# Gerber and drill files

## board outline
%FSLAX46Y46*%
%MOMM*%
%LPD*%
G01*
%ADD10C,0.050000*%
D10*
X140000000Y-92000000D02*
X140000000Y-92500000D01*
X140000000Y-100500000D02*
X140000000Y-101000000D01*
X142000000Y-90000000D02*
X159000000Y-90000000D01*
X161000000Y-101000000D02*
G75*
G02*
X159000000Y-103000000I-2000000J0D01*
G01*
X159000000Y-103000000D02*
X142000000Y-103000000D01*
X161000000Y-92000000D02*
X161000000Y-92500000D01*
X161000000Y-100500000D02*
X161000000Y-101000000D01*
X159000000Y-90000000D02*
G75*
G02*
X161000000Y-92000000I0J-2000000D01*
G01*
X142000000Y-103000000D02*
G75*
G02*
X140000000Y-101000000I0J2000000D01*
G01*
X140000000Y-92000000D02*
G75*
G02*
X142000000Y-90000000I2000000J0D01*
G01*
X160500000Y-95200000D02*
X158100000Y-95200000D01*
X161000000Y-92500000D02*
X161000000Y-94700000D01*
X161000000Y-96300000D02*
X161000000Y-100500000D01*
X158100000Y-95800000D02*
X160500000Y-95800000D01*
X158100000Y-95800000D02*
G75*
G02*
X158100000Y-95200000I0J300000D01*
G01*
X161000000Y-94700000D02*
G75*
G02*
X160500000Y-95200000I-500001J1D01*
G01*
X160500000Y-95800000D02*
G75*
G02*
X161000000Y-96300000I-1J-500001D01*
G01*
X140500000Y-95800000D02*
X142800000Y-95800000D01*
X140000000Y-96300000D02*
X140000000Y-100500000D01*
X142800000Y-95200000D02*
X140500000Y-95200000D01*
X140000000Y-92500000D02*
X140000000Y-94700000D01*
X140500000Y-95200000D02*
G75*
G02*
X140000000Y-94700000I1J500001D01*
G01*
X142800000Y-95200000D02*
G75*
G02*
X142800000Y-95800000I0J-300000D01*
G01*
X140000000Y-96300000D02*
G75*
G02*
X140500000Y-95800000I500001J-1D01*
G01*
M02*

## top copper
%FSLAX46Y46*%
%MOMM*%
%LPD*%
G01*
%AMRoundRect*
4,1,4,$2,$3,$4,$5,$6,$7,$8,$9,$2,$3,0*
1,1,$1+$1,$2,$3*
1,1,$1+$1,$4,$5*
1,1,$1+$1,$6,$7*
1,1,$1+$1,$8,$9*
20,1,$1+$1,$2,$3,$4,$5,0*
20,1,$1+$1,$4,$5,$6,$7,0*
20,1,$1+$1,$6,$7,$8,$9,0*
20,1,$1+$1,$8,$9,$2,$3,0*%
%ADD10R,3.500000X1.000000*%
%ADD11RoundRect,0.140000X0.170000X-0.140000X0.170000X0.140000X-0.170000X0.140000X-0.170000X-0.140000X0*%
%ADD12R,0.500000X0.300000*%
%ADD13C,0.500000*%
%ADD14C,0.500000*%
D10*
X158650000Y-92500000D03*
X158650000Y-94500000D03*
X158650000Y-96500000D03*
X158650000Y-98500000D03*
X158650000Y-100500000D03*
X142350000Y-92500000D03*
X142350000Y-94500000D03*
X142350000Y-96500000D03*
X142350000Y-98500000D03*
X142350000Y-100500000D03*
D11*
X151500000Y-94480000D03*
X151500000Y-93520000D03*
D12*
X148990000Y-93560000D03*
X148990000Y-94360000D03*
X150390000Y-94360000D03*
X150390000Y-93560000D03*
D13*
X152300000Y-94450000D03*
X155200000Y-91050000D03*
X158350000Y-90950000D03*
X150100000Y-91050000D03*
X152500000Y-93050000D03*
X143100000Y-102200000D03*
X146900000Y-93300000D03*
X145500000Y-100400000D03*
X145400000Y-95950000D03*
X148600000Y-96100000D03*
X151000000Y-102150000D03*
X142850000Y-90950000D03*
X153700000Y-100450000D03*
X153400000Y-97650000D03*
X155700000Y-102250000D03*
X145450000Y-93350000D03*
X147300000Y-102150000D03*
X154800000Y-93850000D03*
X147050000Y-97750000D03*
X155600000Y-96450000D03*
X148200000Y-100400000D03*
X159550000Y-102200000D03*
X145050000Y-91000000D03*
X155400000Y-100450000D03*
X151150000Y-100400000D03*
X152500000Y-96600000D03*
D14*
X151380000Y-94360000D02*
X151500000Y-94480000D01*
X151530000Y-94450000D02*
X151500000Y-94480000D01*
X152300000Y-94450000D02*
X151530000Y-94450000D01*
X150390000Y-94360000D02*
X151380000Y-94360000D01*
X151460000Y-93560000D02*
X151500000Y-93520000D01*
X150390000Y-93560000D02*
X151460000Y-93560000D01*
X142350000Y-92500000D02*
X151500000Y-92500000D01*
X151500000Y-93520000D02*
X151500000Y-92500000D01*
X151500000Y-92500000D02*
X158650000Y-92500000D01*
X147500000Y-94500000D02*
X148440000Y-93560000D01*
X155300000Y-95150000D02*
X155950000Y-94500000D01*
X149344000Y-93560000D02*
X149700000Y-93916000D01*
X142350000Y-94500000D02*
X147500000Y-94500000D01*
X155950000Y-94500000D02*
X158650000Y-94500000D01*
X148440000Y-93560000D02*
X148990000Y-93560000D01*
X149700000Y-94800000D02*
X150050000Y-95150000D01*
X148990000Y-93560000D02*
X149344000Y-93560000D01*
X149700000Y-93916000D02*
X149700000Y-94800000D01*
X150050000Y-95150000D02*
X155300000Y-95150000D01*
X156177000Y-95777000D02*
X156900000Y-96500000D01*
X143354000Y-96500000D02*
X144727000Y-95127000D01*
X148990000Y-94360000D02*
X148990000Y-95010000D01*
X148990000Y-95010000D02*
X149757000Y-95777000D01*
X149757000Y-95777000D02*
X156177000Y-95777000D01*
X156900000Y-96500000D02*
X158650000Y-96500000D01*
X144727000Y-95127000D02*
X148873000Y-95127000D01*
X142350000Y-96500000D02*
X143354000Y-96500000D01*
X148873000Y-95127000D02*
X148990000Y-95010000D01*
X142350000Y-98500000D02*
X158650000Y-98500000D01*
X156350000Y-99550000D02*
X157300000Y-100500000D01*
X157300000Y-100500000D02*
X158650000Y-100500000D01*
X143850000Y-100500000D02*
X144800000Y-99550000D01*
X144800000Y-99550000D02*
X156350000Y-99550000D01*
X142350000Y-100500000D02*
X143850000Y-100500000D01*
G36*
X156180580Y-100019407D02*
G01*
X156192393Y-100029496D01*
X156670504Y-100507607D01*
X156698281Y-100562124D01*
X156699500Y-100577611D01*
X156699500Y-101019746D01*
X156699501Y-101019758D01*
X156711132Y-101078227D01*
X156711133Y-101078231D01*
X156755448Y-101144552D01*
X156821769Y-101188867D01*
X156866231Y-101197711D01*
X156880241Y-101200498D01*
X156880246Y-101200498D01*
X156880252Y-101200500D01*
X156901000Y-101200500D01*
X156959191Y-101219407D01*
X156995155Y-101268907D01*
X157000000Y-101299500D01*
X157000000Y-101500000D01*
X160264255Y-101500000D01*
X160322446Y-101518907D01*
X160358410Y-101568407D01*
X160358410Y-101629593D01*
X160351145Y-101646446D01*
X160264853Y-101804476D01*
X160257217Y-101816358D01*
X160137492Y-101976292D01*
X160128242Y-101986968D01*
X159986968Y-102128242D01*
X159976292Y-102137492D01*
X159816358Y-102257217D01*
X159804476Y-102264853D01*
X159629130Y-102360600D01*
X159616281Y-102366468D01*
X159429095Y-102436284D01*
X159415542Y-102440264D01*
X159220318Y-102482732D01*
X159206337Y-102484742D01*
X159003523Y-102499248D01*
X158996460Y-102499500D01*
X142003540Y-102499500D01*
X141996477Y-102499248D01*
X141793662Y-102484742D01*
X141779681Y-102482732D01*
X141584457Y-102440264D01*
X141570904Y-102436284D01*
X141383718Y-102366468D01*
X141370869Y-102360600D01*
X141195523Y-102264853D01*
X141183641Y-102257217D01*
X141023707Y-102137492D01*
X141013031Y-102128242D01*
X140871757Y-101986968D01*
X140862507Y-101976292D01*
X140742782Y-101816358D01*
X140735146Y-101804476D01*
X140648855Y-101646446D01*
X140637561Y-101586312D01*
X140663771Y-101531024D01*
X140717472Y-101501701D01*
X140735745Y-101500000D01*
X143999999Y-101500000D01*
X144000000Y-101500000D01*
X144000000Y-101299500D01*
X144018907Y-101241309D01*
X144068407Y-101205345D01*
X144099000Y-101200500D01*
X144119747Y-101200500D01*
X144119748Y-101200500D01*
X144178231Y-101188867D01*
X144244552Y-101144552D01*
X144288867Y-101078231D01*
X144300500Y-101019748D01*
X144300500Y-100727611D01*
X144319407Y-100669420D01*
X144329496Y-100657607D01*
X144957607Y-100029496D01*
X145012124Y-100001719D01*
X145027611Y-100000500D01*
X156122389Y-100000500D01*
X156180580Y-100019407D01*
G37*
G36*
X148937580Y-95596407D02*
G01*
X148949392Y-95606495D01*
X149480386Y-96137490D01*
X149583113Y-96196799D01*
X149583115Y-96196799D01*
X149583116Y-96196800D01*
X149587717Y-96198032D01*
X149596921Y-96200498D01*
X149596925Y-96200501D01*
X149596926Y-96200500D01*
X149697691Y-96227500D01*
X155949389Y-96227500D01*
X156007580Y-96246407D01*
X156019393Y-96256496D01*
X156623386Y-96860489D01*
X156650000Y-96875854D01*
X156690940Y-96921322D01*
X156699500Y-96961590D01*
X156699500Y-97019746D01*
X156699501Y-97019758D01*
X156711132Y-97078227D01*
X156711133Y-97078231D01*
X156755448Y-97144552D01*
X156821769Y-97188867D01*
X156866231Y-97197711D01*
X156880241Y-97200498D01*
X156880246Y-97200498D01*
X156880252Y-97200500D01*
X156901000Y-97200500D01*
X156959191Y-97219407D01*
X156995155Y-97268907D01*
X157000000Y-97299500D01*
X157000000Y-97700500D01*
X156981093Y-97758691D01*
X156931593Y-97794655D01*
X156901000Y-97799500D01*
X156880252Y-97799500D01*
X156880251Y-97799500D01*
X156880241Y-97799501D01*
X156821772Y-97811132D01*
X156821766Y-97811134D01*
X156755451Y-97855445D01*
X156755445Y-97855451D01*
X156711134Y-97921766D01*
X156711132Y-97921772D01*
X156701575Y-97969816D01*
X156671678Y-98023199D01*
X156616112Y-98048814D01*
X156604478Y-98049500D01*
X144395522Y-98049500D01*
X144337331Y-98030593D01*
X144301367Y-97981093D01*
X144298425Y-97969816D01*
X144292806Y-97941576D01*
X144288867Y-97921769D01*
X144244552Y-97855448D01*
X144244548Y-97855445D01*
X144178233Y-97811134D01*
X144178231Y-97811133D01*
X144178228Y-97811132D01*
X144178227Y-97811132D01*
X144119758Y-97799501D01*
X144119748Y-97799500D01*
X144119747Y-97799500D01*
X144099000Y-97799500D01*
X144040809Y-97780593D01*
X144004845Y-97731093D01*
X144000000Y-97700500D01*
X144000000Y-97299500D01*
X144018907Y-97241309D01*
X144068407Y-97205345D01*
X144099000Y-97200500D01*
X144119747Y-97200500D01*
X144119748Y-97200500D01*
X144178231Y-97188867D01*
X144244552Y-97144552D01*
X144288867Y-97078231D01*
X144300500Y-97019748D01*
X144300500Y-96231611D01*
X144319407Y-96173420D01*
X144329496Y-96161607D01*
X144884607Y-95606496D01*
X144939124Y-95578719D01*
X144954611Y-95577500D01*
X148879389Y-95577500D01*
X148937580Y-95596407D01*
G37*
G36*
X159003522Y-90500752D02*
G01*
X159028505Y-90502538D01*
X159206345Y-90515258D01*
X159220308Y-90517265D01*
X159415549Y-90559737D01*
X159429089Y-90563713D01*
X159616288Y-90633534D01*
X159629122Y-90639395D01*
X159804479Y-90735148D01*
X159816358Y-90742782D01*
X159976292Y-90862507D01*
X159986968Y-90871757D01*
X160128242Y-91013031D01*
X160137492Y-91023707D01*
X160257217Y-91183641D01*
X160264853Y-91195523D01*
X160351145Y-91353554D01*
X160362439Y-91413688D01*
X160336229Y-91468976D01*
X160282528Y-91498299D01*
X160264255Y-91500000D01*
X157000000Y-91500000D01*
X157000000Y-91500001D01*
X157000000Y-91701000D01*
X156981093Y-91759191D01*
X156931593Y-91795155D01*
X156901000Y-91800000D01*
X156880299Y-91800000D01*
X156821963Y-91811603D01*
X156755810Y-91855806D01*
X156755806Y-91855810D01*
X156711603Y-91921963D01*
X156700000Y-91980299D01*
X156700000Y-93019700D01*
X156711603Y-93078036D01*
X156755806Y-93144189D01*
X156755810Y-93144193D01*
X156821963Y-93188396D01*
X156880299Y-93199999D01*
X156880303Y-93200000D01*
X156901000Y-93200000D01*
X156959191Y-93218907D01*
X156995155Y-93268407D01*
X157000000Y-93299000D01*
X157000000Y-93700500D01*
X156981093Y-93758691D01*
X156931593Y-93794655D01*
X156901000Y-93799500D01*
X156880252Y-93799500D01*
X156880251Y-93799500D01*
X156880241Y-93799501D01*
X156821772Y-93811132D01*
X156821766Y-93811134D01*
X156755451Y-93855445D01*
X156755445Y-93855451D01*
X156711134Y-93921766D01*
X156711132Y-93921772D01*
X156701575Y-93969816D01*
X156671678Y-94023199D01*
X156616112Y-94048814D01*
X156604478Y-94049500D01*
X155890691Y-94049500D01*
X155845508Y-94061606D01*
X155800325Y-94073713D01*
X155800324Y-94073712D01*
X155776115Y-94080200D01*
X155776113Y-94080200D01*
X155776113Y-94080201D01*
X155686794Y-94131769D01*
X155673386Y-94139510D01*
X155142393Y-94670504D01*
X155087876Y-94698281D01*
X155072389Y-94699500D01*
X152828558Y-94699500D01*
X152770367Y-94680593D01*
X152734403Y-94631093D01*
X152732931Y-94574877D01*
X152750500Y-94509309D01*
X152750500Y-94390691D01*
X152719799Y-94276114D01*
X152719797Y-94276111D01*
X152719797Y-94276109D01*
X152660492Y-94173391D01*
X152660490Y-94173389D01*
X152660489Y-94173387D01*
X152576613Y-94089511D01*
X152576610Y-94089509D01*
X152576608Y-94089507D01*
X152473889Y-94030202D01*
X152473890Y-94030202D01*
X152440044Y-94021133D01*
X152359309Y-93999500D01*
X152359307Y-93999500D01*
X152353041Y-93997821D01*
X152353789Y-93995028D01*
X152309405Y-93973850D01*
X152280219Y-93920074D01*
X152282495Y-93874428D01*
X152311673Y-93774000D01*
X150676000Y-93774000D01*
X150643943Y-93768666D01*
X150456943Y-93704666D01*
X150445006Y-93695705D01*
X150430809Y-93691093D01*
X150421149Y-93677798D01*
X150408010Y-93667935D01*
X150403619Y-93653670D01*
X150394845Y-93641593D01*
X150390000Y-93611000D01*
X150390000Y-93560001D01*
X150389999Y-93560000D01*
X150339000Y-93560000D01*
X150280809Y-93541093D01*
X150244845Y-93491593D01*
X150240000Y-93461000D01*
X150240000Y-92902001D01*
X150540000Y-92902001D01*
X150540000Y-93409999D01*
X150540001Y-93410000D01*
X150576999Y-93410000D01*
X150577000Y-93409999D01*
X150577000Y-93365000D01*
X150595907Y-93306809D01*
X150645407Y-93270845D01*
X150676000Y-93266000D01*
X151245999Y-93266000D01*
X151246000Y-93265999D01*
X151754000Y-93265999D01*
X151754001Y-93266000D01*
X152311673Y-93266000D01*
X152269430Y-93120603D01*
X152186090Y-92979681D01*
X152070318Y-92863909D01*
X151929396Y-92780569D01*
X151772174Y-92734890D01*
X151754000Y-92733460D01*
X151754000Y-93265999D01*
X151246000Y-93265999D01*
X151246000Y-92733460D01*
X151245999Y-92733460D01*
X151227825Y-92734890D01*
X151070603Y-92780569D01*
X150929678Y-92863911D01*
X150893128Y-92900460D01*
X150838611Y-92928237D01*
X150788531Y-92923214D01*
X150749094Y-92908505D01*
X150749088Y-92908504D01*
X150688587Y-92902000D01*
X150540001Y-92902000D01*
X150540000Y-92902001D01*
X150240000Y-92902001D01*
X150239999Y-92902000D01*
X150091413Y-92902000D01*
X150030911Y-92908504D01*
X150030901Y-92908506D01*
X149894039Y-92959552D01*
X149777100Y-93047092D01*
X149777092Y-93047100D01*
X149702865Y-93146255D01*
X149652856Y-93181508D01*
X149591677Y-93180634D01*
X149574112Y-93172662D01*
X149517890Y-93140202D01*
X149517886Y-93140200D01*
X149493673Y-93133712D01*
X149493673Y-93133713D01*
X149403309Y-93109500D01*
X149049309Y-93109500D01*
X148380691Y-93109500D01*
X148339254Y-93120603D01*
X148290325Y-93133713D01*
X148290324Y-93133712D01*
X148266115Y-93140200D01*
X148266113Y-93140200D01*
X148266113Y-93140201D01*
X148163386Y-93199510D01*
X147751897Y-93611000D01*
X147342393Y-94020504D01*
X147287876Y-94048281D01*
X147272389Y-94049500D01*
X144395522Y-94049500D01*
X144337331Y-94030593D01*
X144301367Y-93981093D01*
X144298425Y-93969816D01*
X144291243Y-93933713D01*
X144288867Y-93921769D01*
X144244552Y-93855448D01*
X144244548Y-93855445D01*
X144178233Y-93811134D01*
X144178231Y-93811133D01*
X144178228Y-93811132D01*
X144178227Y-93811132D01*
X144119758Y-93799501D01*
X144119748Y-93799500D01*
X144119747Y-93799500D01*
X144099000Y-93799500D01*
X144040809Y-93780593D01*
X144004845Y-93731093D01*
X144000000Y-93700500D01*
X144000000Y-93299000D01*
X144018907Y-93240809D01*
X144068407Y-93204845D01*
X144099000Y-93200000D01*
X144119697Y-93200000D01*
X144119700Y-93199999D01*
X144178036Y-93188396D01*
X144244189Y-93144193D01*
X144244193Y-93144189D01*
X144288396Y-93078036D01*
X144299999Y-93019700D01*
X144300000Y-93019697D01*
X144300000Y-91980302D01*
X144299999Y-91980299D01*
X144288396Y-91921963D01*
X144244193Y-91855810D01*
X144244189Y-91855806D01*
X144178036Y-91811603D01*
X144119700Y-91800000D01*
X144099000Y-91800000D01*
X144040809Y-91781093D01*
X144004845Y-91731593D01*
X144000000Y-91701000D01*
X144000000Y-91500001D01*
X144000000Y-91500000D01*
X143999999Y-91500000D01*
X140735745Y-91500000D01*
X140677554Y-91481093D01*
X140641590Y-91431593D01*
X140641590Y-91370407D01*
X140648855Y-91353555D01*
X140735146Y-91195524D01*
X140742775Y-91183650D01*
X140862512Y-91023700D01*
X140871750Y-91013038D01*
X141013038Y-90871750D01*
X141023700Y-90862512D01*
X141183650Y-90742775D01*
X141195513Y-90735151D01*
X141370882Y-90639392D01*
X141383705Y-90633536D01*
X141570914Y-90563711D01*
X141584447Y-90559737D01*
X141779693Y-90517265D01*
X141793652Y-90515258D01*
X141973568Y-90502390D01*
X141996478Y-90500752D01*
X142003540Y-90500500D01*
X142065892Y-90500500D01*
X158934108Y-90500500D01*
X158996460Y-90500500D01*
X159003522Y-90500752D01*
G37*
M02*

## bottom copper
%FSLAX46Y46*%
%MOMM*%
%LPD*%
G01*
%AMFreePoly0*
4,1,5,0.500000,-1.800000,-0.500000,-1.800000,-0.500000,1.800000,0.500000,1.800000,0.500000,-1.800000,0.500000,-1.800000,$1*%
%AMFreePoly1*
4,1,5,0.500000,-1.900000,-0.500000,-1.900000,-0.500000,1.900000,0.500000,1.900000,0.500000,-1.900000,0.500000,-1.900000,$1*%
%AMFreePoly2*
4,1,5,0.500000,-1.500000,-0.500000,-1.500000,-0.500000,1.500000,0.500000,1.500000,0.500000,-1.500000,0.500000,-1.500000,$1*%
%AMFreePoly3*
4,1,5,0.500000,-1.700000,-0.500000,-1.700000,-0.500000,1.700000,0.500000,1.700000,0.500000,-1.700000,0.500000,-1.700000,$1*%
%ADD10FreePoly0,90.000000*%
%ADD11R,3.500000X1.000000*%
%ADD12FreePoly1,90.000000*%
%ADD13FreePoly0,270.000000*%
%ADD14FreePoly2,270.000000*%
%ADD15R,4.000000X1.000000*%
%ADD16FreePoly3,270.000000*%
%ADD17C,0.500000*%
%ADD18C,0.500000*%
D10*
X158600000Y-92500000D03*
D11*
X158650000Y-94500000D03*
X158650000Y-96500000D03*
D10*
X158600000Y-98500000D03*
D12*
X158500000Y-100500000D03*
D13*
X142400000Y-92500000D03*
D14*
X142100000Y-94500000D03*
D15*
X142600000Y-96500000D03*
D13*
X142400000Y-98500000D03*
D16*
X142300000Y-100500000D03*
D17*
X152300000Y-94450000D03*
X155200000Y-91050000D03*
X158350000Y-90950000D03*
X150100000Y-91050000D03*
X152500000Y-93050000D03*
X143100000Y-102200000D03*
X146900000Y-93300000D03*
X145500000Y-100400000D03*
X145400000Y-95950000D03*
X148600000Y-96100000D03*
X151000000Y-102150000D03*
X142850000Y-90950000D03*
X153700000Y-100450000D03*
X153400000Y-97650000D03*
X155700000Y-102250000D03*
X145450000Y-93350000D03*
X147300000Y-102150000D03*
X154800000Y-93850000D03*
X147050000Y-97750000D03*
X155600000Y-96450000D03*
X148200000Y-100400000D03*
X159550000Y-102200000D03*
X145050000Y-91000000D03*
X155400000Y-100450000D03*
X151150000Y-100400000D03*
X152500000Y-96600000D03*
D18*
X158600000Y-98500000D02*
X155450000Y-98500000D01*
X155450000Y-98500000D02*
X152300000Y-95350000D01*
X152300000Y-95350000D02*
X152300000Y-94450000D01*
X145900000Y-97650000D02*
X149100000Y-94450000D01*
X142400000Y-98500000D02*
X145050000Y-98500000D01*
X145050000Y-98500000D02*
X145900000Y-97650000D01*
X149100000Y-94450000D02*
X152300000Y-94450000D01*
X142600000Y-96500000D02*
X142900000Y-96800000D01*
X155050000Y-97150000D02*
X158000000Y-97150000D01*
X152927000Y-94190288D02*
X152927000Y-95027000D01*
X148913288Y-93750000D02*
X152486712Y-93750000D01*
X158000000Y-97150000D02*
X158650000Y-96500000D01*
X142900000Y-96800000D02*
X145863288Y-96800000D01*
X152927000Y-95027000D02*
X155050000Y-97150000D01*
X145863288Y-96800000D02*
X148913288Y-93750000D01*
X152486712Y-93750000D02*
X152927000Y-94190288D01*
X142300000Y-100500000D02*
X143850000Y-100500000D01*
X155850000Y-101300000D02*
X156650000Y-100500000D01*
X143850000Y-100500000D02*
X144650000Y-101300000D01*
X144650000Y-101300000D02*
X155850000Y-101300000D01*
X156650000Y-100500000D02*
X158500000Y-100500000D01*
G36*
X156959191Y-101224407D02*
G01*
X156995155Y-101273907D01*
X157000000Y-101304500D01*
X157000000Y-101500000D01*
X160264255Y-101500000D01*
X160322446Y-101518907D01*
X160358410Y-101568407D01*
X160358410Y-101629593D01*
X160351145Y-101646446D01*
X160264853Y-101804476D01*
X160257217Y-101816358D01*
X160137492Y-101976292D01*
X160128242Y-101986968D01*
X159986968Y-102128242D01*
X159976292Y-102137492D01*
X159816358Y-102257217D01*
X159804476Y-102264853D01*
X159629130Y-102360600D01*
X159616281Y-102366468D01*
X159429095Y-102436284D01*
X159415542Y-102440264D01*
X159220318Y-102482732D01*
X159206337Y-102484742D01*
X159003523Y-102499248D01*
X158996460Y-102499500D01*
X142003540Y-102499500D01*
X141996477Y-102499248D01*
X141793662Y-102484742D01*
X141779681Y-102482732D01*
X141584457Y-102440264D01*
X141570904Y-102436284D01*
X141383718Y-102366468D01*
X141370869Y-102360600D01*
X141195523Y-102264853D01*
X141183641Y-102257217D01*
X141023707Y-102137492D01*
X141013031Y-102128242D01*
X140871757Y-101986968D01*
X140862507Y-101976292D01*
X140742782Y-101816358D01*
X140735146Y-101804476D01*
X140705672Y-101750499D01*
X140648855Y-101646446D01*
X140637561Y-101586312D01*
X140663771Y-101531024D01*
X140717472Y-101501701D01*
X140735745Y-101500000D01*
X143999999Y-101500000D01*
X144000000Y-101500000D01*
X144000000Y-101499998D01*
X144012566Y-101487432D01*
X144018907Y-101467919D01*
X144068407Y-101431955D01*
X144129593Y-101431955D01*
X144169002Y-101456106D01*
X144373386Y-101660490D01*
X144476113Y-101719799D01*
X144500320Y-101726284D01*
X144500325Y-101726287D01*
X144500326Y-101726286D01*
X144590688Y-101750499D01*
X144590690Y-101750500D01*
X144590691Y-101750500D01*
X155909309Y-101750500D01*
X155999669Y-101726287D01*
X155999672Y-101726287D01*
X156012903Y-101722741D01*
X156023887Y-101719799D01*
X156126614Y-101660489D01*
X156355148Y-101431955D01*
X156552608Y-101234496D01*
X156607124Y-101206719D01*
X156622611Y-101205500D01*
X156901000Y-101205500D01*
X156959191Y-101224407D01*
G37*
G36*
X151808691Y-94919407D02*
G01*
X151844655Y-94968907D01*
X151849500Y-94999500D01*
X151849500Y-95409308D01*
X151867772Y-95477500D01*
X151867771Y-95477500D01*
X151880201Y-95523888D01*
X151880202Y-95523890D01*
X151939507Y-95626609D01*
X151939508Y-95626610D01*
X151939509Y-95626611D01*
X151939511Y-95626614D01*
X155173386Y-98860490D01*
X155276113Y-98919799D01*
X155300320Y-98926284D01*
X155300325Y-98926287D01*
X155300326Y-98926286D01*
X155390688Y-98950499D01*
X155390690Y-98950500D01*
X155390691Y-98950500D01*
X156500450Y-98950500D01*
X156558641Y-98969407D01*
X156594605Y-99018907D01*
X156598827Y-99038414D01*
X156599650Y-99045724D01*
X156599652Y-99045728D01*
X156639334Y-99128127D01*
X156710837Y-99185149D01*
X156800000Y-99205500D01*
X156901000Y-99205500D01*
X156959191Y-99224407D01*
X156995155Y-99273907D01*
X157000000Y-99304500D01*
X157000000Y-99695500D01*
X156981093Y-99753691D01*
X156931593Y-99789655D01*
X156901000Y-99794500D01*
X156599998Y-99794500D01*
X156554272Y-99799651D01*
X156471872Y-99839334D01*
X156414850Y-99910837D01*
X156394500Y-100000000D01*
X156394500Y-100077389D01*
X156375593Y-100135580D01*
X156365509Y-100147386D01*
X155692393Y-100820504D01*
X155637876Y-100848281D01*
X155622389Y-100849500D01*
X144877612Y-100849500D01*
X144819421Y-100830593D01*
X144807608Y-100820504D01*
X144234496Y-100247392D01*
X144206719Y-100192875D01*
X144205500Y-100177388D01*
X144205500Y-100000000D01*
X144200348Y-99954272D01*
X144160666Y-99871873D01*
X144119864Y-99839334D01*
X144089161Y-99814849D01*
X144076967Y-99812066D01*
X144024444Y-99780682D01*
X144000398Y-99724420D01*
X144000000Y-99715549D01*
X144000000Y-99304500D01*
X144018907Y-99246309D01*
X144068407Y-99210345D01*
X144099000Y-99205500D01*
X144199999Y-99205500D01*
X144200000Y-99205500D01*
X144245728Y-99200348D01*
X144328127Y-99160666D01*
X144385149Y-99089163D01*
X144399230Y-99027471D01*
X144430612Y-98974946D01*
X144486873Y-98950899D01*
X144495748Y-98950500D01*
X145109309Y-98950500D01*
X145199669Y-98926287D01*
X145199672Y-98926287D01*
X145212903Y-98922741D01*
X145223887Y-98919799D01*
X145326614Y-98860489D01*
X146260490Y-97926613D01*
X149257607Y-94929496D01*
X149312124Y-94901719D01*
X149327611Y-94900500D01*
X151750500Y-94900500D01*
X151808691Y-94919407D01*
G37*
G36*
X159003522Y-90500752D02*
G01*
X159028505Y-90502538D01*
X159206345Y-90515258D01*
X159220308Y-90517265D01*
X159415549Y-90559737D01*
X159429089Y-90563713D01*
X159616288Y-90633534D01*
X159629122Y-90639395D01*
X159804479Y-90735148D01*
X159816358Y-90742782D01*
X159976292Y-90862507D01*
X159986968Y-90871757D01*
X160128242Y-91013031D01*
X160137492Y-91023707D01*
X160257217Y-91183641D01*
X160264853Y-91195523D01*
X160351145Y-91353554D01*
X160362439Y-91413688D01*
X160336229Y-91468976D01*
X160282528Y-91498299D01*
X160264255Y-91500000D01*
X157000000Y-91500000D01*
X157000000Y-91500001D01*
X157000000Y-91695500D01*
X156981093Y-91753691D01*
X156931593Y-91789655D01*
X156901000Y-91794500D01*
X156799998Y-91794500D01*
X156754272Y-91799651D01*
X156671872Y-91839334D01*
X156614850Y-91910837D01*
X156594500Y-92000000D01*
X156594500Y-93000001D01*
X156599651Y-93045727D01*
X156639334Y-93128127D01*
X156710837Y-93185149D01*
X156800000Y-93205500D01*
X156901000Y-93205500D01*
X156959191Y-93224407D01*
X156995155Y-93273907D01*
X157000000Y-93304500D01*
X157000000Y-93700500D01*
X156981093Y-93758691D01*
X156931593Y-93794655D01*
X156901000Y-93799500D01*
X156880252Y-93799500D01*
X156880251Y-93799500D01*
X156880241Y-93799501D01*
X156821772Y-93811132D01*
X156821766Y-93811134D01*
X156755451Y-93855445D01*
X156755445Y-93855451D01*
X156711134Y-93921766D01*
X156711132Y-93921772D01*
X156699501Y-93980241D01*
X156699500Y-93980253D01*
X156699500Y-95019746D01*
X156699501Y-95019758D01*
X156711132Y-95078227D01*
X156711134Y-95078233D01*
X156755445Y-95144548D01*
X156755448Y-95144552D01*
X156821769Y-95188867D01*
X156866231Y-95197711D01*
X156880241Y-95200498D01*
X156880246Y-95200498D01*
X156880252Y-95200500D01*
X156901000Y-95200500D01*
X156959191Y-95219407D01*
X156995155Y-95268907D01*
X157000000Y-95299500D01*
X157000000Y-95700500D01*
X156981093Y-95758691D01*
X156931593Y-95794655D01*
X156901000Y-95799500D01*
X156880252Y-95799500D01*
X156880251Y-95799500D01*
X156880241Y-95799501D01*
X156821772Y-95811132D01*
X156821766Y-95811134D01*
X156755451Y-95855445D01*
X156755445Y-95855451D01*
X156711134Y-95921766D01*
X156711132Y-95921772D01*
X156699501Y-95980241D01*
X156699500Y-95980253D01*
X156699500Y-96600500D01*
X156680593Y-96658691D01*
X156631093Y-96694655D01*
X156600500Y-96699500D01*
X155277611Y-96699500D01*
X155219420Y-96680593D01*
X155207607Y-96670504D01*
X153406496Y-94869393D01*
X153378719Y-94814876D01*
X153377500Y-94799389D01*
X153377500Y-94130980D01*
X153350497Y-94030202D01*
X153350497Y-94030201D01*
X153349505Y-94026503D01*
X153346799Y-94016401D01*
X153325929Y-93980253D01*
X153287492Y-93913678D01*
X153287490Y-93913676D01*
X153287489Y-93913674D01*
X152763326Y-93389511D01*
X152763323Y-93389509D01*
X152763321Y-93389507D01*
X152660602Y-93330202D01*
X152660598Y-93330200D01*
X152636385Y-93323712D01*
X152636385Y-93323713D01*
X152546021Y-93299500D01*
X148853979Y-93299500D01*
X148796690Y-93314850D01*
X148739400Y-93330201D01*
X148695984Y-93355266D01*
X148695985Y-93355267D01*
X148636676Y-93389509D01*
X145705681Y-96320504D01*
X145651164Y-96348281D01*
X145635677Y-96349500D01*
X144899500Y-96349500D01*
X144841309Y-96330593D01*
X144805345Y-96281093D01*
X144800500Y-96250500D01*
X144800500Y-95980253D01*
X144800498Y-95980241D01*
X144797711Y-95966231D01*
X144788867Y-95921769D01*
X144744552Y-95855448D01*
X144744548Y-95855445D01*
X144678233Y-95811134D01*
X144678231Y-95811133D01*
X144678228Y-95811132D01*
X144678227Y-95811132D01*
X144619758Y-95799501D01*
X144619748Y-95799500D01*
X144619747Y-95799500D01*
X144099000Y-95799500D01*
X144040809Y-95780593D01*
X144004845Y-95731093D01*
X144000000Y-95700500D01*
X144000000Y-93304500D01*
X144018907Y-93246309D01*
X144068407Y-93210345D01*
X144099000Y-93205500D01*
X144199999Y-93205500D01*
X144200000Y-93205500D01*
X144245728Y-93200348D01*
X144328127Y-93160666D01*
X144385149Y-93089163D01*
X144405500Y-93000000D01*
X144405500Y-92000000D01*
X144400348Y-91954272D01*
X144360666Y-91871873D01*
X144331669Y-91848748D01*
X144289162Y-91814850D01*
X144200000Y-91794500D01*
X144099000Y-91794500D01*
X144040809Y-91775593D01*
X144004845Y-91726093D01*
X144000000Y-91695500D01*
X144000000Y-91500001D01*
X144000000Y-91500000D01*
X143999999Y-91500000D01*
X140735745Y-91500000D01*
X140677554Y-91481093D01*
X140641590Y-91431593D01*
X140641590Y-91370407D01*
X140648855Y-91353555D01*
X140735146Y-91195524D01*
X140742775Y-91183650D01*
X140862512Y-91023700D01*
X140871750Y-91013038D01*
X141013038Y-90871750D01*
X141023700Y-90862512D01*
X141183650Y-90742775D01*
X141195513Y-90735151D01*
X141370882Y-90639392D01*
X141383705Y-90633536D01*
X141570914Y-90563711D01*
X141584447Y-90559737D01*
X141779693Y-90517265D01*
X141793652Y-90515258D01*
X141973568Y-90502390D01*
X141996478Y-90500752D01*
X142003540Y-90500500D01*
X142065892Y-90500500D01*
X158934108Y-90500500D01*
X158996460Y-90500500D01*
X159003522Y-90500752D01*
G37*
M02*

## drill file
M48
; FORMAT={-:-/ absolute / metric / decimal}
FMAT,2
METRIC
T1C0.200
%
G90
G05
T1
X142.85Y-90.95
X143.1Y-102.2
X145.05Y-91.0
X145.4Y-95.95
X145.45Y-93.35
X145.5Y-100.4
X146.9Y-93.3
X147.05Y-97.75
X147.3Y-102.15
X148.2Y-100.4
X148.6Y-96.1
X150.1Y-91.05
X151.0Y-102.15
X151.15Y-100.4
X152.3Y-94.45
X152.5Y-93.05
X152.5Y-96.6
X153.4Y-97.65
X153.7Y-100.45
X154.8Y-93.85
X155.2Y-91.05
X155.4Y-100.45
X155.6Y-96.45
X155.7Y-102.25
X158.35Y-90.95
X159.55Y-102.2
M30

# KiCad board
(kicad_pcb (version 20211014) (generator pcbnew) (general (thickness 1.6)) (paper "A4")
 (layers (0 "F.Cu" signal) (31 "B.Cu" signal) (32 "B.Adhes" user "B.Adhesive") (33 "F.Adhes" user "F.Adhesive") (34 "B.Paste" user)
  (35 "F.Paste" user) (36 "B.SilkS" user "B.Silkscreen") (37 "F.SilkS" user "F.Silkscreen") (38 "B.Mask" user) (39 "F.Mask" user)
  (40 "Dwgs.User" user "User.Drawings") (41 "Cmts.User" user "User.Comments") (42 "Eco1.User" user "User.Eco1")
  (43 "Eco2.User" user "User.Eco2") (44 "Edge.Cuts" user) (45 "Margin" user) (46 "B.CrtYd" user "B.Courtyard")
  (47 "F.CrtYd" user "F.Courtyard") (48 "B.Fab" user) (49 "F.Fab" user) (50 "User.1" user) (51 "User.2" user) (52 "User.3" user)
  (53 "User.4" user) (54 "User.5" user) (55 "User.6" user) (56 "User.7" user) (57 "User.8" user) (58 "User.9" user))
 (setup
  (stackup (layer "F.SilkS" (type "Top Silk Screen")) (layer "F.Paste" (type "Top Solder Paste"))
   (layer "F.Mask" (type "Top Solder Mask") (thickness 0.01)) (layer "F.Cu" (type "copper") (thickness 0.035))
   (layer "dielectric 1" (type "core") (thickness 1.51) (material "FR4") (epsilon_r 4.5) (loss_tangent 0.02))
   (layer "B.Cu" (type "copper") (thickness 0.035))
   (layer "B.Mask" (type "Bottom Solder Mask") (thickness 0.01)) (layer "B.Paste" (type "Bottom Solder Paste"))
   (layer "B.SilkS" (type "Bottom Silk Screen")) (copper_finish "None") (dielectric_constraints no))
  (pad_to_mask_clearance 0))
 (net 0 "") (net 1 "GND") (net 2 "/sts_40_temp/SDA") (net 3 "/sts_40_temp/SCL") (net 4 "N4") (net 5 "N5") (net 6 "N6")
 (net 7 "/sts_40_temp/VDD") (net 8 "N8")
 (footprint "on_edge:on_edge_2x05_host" (layer "F.Cu") (at 161 96.5 -90)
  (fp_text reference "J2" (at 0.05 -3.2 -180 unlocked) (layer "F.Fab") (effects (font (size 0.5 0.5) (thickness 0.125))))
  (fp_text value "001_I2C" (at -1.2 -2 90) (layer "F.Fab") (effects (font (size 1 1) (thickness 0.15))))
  (fp_line (start -1.3 0.5) (end -1.3 2.9) (layer "Edge.Cuts") (width 0.05))
  (fp_line (start -4 0) (end -1.8 0) (layer "Edge.Cuts") (width 0.05))
  (fp_line (start -0.2 0) (end 4 0) (layer "Edge.Cuts") (width 0.05))
  (fp_line (start -0.7 2.9) (end -0.7 0.5) (layer "Edge.Cuts") (width 0.05))
  (fp_arc (start -0.7 2.9) (mid -1 3.2) (end -1.3 2.9) (layer "Edge.Cuts") (width 0.05))
  (fp_arc (start -1.8 0) (mid -1.446447 0.146447) (end -1.3 0.5) (layer "Edge.Cuts") (width 0.05))
  (fp_arc (start -0.7 0.5) (mid -0.553553 0.146447) (end -0.2 0) (layer "Edge.Cuts") (width 0.05))
  (pad "1" smd rect (at -4 2.35 270) (size 1 3.5) (layers "F.Cu" "F.Mask") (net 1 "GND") (zone_connect 0))
  (pad "2" smd rect (at -2 2.35 270) (size 1 3.5) (layers "F.Cu" "F.Mask") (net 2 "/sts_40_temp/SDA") (zone_connect 0))
  (pad "3" smd rect (at 0 2.35 270) (size 1 3.5) (layers "F.Cu" "F.Mask") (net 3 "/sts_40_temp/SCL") (zone_connect 0))
  (pad "4" smd rect (at 2 2.35 270) (size 1 3.5) (layers "F.Cu" "F.Mask") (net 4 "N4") (zone_connect 0))
  (pad "5" smd rect (at 4 2.35 270) (size 1 3.5) (layers "F.Cu" "F.Mask") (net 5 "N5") (zone_connect 0))
  (pad "6" smd custom (at -4 2.4 90) (size 1 3.6) (layers "B.Cu" "B.Mask") (zone_connect 0) (options (clearance outline) (anchor rect))
   (primitives))
  (pad "7" smd rect (at -2 2.35 90) (size 1 3.5) (layers "B.Cu" "B.Mask") (zone_connect 0))
  (pad "8" smd rect (at 0 2.35 90) (size 1 3.5) (layers "B.Cu" "B.Mask") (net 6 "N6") (zone_connect 0))
  (pad "9" smd custom (at 2 2.4 90) (size 1 3.6) (layers "B.Cu" "B.Mask") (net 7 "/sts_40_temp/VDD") (zone_connect 0)
   (options (clearance outline) (anchor rect)) (primitives))
  (pad "10" smd custom (at 4 2.5 90) (size 1 3.8) (layers "B.Cu" "B.Mask") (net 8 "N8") (zone_connect 0)
   (options (clearance outline) (anchor rect)) (primitives))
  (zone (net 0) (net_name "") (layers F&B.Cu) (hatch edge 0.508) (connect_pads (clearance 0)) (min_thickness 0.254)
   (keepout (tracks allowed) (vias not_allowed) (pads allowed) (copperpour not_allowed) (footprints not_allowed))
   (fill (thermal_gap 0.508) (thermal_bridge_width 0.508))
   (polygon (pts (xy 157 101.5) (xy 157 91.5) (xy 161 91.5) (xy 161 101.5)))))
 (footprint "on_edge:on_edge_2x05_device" (layer "F.Cu") (at 140 96.5 -90)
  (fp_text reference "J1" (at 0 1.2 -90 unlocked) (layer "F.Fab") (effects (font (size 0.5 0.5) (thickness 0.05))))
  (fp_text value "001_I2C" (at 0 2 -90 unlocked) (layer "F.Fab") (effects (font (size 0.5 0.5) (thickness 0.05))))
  (fp_line (start -0.7 -0.5) (end -0.7 -2.8) (layer "Edge.Cuts") (width 0.05))
  (fp_line (start -0.2 0) (end 4 0) (layer "Edge.Cuts") (width 0.05))
  (fp_line (start -1.3 -2.8) (end -1.3 -0.5) (layer "Edge.Cuts") (width 0.05))
  (fp_line (start -4 0) (end -1.8 0) (layer "Edge.Cuts") (width 0.05))
  (fp_arc (start -1.3 -0.5) (mid -1.446447 -0.146447) (end -1.8 0) (layer "Edge.Cuts") (width 0.05))
  (fp_arc (start -1.3 -2.8) (mid -1 -3.1) (end -0.7 -2.8) (layer "Edge.Cuts") (width 0.05))
  (fp_arc (start -0.2 0) (mid -0.553553 -0.146447) (end -0.7 -0.5) (layer "Edge.Cuts") (width 0.05))
  (pad "1" smd rect (at -4 -2.35 90) (size 1 3.5) (layers "F.Cu" "F.Mask") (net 1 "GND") (zone_connect 0))
  (pad "2" smd rect (at -2 -2.35 270) (size 1 3.5) (layers "F.Cu" "F.Mask") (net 2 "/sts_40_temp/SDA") (zone_connect 0))
  (pad "3" smd rect (at 0 -2.35 270) (size 1 3.5) (layers "F.Cu" "F.Mask") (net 3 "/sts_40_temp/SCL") (zone_connect 0))
  (pad "4" smd rect (at 2 -2.35 90) (size 1 3.5) (layers "F.Cu" "F.Mask") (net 4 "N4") (zone_connect 0))
  (pad "5" smd rect (at 4 -2.35 90) (size 1 3.5) (layers "F.Cu" "F.Mask") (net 5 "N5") (zone_connect 0))
  (pad "6" smd custom (at -4 -2.4 270) (size 1 3.6) (layers "B.Cu" "B.Mask") (zone_connect 0) (options (clearance outline) (anchor rect))
   (primitives))
  (pad "7" smd custom (at -2 -2.1 270) (size 1 3) (layers "B.Cu" "B.Mask") (zone_connect 0) (options (clearance outline) (anchor rect))
   (primitives))
  (pad "8" smd rect (at 0 -2.6 270) (size 1 4) (layers "B.Cu" "B.Mask") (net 6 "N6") (zone_connect 0))
  (pad "9" smd custom (at 2 -2.4 270) (size 1 3.6) (layers "B.Cu" "B.Mask") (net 7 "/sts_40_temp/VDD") (zone_connect 0)
   (options (clearance outline) (anchor rect)) (primitives))
  (pad "10" smd custom (at 4 -2.3 270) (size 1 3.4) (layers "B.Cu" "B.Mask") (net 8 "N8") (zone_connect 0)
   (options (clearance outline) (anchor rect)) (primitives))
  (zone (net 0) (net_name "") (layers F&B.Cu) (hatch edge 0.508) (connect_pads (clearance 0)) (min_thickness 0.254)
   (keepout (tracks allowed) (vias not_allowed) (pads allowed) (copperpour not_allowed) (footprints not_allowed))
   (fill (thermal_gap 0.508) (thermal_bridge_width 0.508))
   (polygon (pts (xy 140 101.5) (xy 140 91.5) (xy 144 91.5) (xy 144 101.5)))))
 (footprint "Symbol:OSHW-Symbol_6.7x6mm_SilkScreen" (layer "F.Cu") (at 150.45 99.55)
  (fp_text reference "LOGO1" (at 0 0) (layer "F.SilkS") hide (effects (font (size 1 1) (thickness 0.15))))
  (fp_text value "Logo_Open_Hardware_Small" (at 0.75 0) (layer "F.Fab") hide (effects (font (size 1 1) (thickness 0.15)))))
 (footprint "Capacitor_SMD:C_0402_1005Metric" (layer "F.Cu") (at 151.5 94 90)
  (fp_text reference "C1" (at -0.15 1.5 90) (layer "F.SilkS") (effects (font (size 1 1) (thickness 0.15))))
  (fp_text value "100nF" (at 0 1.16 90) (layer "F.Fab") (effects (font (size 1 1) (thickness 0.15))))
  (pad "1" smd roundrect (at -0.48 0 90) (size 0.56 0.62) (layers "F.Cu" "F.Paste" "F.Mask") (roundrect_rratio 0.25)
   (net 7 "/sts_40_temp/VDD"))
  (pad "2" smd roundrect (at 0.48 0 90) (size 0.56 0.62) (layers "F.Cu" "F.Paste" "F.Mask") (roundrect_rratio 0.25) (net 1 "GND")))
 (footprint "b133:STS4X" (layer "F.Cu") (at 149.69 93.96)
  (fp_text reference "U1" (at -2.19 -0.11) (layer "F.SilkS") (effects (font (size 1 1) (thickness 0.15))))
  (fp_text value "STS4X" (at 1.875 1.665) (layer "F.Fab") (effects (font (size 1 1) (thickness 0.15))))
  (pad "1" smd rect (at -0.7 -0.4) (size 0.5 0.3) (layers "F.Cu" "F.Paste" "F.Mask") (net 2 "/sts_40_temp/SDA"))
  (pad "2" smd rect (at -0.7 0.4) (size 0.5 0.3) (layers "F.Cu" "F.Paste" "F.Mask") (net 3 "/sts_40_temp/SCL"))
  (pad "3" smd rect (at 0.7 0.4) (size 0.5 0.3) (layers "F.Cu" "F.Paste" "F.Mask") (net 7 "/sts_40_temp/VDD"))
  (pad "4" smd rect (at 0.7 -0.4) (size 0.5 0.3) (layers "F.Cu" "F.Paste" "F.Mask") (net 1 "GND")))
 (gr_line (start 140 92) (end 140 92.5) (layer "Edge.Cuts") (width 0.05))
 (gr_line (start 140 100.5) (end 140 101) (layer "Edge.Cuts") (width 0.05))
 (gr_line (start 142 90) (end 159 90) (layer "Edge.Cuts") (width 0.05))
 (gr_arc (start 161 101) (mid 160.414214 102.414214) (end 159 103) (layer "Edge.Cuts") (width 0.05))
 (gr_line (start 159 103) (end 142 103) (layer "Edge.Cuts") (width 0.05))
 (gr_line (start 161 92) (end 161 92.5) (layer "Edge.Cuts") (width 0.05))
 (gr_line (start 161 100.5) (end 161 101) (layer "Edge.Cuts") (width 0.05))
 (gr_arc (start 159 90) (mid 160.414214 90.585786) (end 161 92) (layer "Edge.Cuts") (width 0.05))
 (gr_arc (start 142 103) (mid 140.585786 102.414214) (end 140 101) (layer "Edge.Cuts") (width 0.05))
 (gr_arc (start 140 92) (mid 140.585786 90.585786) (end 142 90) (layer "Edge.Cuts") (width 0.05))
 (segment (start 151.38 94.36) (end 151.5 94.48) (width 0.5) (layer "F.Cu") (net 7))
 (segment (start 151.53 94.45) (end 151.5 94.48) (width 0.5) (layer "F.Cu") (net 7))
 (segment (start 152.3 94.45) (end 151.53 94.45) (width 0.5) (layer "F.Cu") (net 7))
 (segment (start 150.39 94.36) (end 151.38 94.36) (width 0.5) (layer "F.Cu") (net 7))
 (via (at 152.3 94.45) (size 0.5) (drill 0.2) (layers "F.Cu" "B.Cu") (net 7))
 (segment (start 158.6 98.5) (end 155.45 98.5) (width 0.5) (layer "B.Cu") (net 7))
 (segment (start 155.45 98.5) (end 152.3 95.35) (width 0.5) (layer "B.Cu") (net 7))
 (segment (start 152.3 95.35) (end 152.3 94.45) (width 0.5) (layer "B.Cu") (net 7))
 (segment (start 145.9 97.65) (end 149.1 94.45) (width 0.5) (layer "B.Cu") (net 7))
 (segment (start 142.4 98.5) (end 145.05 98.5) (width 0.5) (layer "B.Cu") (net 7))
 (segment (start 145.05 98.5) (end 145.9 97.65) (width 0.5) (layer "B.Cu") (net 7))
 (segment (start 149.1 94.45) (end 152.3 94.45) (width 0.5) (layer "B.Cu") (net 7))
 (segment (start 151.46 93.56) (end 151.5 93.52) (width 0.5) (layer "F.Cu") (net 1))
 (segment (start 150.39 93.56) (end 151.46 93.56) (width 0.5) (layer "F.Cu") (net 1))
 (segment (start 142.35 92.5) (end 151.5 92.5) (width 0.5) (layer "F.Cu") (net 1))
 (segment (start 151.5 93.52) (end 151.5 92.5) (width 0.5) (layer "F.Cu") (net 1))
 (segment (start 151.5 92.5) (end 158.65 92.5) (width 0.5) (layer "F.Cu") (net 1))
 (via (at 155.2 91.05) (size 0.5) (drill 0.2) (layers "F.Cu" "B.Cu") (free) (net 1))
 (via (at 158.35 90.95) (size 0.5) (drill 0.2) (layers "F.Cu" "B.Cu") (free) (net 1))
 (via (at 150.1 91.05) (size 0.5) (drill 0.2) (layers "F.Cu" "B.Cu") (free) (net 1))
 (via (at 152.5 93.05) (size 0.5) (drill 0.2) (layers "F.Cu" "B.Cu") (free) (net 1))
 (via (at 143.1 102.2) (size 0.5) (drill 0.2) (layers "F.Cu" "B.Cu") (free) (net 1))
 (via (at 146.9 93.3) (size 0.5) (drill 0.2) (layers "F.Cu" "B.Cu") (free) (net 1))
 (via (at 145.5 100.4) (size 0.5) (drill 0.2) (layers "F.Cu" "B.Cu") (free) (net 1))
 (via (at 145.4 95.95) (size 0.5) (drill 0.2) (layers "F.Cu" "B.Cu") (free) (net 1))
 (via (at 148.6 96.1) (size 0.5) (drill 0.2) (layers "F.Cu" "B.Cu") (free) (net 1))
 (via (at 151 102.15) (size 0.5) (drill 0.2) (layers "F.Cu" "B.Cu") (free) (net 1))
 (via (at 142.85 90.95) (size 0.5) (drill 0.2) (layers "F.Cu" "B.Cu") (free) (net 1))
 (via (at 153.7 100.45) (size 0.5) (drill 0.2) (layers "F.Cu" "B.Cu") (free) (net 1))
 (via (at 153.4 97.65) (size 0.5) (drill 0.2) (layers "F.Cu" "B.Cu") (free) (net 1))
 (via (at 155.7 102.25) (size 0.5) (drill 0.2) (layers "F.Cu" "B.Cu") (free) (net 1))
 (via (at 145.45 93.35) (size 0.5) (drill 0.2) (layers "F.Cu" "B.Cu") (free) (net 1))
 (via (at 147.3 102.15) (size 0.5) (drill 0.2) (layers "F.Cu" "B.Cu") (free) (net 1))
 (via (at 154.8 93.85) (size 0.5) (drill 0.2) (layers "F.Cu" "B.Cu") (free) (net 1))
 (via (at 147.05 97.75) (size 0.5) (drill 0.2) (layers "F.Cu" "B.Cu") (free) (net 1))
 (via (at 155.6 96.45) (size 0.5) (drill 0.2) (layers "F.Cu" "B.Cu") (free) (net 1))
 (via (at 148.2 100.4) (size 0.5) (drill 0.2) (layers "F.Cu" "B.Cu") (free) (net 1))
 (via (at 159.55 102.2) (size 0.5) (drill 0.2) (layers "F.Cu" "B.Cu") (free) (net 1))
 (via (at 145.05 91) (size 0.5) (drill 0.2) (layers "F.Cu" "B.Cu") (free) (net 1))
 (via (at 155.4 100.45) (size 0.5) (drill 0.2) (layers "F.Cu" "B.Cu") (free) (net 1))
 (via (at 151.15 100.4) (size 0.5) (drill 0.2) (layers "F.Cu" "B.Cu") (free) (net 1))
 (via (at 152.5 96.6) (size 0.5) (drill 0.2) (layers "F.Cu" "B.Cu") (free) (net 1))
 (segment (start 147.5 94.5) (end 148.44 93.56) (width 0.5) (layer "F.Cu") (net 2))
 (segment (start 155.3 95.15) (end 155.95 94.5) (width 0.5) (layer "F.Cu") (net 2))
 (segment (start 149.344 93.56) (end 149.7 93.916) (width 0.5) (layer "F.Cu") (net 2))
 (segment (start 142.35 94.5) (end 147.5 94.5) (width 0.5) (layer "F.Cu") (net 2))
 (segment (start 155.95 94.5) (end 158.65 94.5) (width 0.5) (layer "F.Cu") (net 2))
 (segment (start 148.44 93.56) (end 148.99 93.56) (width 0.5) (layer "F.Cu") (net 2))
 (segment (start 149.7 94.8) (end 150.05 95.15) (width 0.5) (layer "F.Cu") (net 2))
 (segment (start 148.99 93.56) (end 149.344 93.56) (width 0.5) (layer "F.Cu") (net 2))
 (segment (start 149.7 93.916) (end 149.7 94.8) (width 0.5) (layer "F.Cu") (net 2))
 (segment (start 150.05 95.15) (end 155.3 95.15) (width 0.5) (layer "F.Cu") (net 2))
 (segment (start 156.177 95.777) (end 156.9 96.5) (width 0.5) (layer "F.Cu") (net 3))
 (segment (start 143.354 96.5) (end 144.727 95.127) (width 0.5) (layer "F.Cu") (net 3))
 (segment (start 148.99 94.36) (end 148.99 95.01) (width 0.5) (layer "F.Cu") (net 3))
 (segment (start 148.99 95.01) (end 149.757 95.777) (width 0.5) (layer "F.Cu") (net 3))
 (segment (start 149.757 95.777) (end 156.177 95.777) (width 0.5) (layer "F.Cu") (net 3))
 (segment (start 156.9 96.5) (end 158.65 96.5) (width 0.5) (layer "F.Cu") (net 3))
 (segment (start 144.727 95.127) (end 148.873 95.127) (width 0.5) (layer "F.Cu") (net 3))
 (segment (start 142.35 96.5) (end 143.354 96.5) (width 0.5) (layer "F.Cu") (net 3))
 (segment (start 148.873 95.127) (end 148.99 95.01) (width 0.5) (layer "F.Cu") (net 3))
 (segment (start 142.35 98.5) (end 158.65 98.5) (width 0.5) (layer "F.Cu") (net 4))
 (segment (start 156.35 99.55) (end 157.3 100.5) (width 0.5) (layer "F.Cu") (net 5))
 (segment (start 157.3 100.5) (end 158.65 100.5) (width 0.5) (layer "F.Cu") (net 5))
 (segment (start 143.85 100.5) (end 144.8 99.55) (width 0.5) (layer "F.Cu") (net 5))
 (segment (start 144.8 99.55) (end 156.35 99.55) (width 0.5) (layer "F.Cu") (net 5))
 (segment (start 142.35 100.5) (end 143.85 100.5) (width 0.5) (layer "F.Cu") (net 5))
 (segment (start 142.6 96.5) (end 142.9 96.8) (width 0.5) (layer "B.Cu") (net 6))
 (segment (start 155.05 97.15) (end 158 97.15) (width 0.5) (layer "B.Cu") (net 6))
 (segment (start 152.927 94.190288) (end 152.927 95.027) (width 0.5) (layer "B.Cu") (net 6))
 (segment (start 148.913288 93.75) (end 152.486712 93.75) (width 0.5) (layer "B.Cu") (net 6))
 (segment (start 158 97.15) (end 158.65 96.5) (width 0.5) (layer "B.Cu") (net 6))
 (segment (start 142.9 96.8) (end 145.863288 96.8) (width 0.5) (layer "B.Cu") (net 6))
 (segment (start 152.927 95.027) (end 155.05 97.15) (width 0.5) (layer "B.Cu") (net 6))
 (segment (start 145.863288 96.8) (end 148.913288 93.75) (width 0.5) (layer "B.Cu") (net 6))
 (segment (start 152.486712 93.75) (end 152.927 94.190288) (width 0.5) (layer "B.Cu") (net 6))
 (segment (start 142.3 100.5) (end 143.85 100.5) (width 0.5) (layer "B.Cu") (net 8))
 (segment (start 155.85 101.3) (end 156.65 100.5) (width 0.5) (layer "B.Cu") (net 8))
 (segment (start 143.85 100.5) (end 144.65 101.3) (width 0.5) (layer "B.Cu") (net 8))
 (segment (start 144.65 101.3) (end 155.85 101.3) (width 0.5) (layer "B.Cu") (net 8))
 (segment (start 156.65 100.5) (end 158.5 100.5) (width 0.5) (layer "B.Cu") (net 8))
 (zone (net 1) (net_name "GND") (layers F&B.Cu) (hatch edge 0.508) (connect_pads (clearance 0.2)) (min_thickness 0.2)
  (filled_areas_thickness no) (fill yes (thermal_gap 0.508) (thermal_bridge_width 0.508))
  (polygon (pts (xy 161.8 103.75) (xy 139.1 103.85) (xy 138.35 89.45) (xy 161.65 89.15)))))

